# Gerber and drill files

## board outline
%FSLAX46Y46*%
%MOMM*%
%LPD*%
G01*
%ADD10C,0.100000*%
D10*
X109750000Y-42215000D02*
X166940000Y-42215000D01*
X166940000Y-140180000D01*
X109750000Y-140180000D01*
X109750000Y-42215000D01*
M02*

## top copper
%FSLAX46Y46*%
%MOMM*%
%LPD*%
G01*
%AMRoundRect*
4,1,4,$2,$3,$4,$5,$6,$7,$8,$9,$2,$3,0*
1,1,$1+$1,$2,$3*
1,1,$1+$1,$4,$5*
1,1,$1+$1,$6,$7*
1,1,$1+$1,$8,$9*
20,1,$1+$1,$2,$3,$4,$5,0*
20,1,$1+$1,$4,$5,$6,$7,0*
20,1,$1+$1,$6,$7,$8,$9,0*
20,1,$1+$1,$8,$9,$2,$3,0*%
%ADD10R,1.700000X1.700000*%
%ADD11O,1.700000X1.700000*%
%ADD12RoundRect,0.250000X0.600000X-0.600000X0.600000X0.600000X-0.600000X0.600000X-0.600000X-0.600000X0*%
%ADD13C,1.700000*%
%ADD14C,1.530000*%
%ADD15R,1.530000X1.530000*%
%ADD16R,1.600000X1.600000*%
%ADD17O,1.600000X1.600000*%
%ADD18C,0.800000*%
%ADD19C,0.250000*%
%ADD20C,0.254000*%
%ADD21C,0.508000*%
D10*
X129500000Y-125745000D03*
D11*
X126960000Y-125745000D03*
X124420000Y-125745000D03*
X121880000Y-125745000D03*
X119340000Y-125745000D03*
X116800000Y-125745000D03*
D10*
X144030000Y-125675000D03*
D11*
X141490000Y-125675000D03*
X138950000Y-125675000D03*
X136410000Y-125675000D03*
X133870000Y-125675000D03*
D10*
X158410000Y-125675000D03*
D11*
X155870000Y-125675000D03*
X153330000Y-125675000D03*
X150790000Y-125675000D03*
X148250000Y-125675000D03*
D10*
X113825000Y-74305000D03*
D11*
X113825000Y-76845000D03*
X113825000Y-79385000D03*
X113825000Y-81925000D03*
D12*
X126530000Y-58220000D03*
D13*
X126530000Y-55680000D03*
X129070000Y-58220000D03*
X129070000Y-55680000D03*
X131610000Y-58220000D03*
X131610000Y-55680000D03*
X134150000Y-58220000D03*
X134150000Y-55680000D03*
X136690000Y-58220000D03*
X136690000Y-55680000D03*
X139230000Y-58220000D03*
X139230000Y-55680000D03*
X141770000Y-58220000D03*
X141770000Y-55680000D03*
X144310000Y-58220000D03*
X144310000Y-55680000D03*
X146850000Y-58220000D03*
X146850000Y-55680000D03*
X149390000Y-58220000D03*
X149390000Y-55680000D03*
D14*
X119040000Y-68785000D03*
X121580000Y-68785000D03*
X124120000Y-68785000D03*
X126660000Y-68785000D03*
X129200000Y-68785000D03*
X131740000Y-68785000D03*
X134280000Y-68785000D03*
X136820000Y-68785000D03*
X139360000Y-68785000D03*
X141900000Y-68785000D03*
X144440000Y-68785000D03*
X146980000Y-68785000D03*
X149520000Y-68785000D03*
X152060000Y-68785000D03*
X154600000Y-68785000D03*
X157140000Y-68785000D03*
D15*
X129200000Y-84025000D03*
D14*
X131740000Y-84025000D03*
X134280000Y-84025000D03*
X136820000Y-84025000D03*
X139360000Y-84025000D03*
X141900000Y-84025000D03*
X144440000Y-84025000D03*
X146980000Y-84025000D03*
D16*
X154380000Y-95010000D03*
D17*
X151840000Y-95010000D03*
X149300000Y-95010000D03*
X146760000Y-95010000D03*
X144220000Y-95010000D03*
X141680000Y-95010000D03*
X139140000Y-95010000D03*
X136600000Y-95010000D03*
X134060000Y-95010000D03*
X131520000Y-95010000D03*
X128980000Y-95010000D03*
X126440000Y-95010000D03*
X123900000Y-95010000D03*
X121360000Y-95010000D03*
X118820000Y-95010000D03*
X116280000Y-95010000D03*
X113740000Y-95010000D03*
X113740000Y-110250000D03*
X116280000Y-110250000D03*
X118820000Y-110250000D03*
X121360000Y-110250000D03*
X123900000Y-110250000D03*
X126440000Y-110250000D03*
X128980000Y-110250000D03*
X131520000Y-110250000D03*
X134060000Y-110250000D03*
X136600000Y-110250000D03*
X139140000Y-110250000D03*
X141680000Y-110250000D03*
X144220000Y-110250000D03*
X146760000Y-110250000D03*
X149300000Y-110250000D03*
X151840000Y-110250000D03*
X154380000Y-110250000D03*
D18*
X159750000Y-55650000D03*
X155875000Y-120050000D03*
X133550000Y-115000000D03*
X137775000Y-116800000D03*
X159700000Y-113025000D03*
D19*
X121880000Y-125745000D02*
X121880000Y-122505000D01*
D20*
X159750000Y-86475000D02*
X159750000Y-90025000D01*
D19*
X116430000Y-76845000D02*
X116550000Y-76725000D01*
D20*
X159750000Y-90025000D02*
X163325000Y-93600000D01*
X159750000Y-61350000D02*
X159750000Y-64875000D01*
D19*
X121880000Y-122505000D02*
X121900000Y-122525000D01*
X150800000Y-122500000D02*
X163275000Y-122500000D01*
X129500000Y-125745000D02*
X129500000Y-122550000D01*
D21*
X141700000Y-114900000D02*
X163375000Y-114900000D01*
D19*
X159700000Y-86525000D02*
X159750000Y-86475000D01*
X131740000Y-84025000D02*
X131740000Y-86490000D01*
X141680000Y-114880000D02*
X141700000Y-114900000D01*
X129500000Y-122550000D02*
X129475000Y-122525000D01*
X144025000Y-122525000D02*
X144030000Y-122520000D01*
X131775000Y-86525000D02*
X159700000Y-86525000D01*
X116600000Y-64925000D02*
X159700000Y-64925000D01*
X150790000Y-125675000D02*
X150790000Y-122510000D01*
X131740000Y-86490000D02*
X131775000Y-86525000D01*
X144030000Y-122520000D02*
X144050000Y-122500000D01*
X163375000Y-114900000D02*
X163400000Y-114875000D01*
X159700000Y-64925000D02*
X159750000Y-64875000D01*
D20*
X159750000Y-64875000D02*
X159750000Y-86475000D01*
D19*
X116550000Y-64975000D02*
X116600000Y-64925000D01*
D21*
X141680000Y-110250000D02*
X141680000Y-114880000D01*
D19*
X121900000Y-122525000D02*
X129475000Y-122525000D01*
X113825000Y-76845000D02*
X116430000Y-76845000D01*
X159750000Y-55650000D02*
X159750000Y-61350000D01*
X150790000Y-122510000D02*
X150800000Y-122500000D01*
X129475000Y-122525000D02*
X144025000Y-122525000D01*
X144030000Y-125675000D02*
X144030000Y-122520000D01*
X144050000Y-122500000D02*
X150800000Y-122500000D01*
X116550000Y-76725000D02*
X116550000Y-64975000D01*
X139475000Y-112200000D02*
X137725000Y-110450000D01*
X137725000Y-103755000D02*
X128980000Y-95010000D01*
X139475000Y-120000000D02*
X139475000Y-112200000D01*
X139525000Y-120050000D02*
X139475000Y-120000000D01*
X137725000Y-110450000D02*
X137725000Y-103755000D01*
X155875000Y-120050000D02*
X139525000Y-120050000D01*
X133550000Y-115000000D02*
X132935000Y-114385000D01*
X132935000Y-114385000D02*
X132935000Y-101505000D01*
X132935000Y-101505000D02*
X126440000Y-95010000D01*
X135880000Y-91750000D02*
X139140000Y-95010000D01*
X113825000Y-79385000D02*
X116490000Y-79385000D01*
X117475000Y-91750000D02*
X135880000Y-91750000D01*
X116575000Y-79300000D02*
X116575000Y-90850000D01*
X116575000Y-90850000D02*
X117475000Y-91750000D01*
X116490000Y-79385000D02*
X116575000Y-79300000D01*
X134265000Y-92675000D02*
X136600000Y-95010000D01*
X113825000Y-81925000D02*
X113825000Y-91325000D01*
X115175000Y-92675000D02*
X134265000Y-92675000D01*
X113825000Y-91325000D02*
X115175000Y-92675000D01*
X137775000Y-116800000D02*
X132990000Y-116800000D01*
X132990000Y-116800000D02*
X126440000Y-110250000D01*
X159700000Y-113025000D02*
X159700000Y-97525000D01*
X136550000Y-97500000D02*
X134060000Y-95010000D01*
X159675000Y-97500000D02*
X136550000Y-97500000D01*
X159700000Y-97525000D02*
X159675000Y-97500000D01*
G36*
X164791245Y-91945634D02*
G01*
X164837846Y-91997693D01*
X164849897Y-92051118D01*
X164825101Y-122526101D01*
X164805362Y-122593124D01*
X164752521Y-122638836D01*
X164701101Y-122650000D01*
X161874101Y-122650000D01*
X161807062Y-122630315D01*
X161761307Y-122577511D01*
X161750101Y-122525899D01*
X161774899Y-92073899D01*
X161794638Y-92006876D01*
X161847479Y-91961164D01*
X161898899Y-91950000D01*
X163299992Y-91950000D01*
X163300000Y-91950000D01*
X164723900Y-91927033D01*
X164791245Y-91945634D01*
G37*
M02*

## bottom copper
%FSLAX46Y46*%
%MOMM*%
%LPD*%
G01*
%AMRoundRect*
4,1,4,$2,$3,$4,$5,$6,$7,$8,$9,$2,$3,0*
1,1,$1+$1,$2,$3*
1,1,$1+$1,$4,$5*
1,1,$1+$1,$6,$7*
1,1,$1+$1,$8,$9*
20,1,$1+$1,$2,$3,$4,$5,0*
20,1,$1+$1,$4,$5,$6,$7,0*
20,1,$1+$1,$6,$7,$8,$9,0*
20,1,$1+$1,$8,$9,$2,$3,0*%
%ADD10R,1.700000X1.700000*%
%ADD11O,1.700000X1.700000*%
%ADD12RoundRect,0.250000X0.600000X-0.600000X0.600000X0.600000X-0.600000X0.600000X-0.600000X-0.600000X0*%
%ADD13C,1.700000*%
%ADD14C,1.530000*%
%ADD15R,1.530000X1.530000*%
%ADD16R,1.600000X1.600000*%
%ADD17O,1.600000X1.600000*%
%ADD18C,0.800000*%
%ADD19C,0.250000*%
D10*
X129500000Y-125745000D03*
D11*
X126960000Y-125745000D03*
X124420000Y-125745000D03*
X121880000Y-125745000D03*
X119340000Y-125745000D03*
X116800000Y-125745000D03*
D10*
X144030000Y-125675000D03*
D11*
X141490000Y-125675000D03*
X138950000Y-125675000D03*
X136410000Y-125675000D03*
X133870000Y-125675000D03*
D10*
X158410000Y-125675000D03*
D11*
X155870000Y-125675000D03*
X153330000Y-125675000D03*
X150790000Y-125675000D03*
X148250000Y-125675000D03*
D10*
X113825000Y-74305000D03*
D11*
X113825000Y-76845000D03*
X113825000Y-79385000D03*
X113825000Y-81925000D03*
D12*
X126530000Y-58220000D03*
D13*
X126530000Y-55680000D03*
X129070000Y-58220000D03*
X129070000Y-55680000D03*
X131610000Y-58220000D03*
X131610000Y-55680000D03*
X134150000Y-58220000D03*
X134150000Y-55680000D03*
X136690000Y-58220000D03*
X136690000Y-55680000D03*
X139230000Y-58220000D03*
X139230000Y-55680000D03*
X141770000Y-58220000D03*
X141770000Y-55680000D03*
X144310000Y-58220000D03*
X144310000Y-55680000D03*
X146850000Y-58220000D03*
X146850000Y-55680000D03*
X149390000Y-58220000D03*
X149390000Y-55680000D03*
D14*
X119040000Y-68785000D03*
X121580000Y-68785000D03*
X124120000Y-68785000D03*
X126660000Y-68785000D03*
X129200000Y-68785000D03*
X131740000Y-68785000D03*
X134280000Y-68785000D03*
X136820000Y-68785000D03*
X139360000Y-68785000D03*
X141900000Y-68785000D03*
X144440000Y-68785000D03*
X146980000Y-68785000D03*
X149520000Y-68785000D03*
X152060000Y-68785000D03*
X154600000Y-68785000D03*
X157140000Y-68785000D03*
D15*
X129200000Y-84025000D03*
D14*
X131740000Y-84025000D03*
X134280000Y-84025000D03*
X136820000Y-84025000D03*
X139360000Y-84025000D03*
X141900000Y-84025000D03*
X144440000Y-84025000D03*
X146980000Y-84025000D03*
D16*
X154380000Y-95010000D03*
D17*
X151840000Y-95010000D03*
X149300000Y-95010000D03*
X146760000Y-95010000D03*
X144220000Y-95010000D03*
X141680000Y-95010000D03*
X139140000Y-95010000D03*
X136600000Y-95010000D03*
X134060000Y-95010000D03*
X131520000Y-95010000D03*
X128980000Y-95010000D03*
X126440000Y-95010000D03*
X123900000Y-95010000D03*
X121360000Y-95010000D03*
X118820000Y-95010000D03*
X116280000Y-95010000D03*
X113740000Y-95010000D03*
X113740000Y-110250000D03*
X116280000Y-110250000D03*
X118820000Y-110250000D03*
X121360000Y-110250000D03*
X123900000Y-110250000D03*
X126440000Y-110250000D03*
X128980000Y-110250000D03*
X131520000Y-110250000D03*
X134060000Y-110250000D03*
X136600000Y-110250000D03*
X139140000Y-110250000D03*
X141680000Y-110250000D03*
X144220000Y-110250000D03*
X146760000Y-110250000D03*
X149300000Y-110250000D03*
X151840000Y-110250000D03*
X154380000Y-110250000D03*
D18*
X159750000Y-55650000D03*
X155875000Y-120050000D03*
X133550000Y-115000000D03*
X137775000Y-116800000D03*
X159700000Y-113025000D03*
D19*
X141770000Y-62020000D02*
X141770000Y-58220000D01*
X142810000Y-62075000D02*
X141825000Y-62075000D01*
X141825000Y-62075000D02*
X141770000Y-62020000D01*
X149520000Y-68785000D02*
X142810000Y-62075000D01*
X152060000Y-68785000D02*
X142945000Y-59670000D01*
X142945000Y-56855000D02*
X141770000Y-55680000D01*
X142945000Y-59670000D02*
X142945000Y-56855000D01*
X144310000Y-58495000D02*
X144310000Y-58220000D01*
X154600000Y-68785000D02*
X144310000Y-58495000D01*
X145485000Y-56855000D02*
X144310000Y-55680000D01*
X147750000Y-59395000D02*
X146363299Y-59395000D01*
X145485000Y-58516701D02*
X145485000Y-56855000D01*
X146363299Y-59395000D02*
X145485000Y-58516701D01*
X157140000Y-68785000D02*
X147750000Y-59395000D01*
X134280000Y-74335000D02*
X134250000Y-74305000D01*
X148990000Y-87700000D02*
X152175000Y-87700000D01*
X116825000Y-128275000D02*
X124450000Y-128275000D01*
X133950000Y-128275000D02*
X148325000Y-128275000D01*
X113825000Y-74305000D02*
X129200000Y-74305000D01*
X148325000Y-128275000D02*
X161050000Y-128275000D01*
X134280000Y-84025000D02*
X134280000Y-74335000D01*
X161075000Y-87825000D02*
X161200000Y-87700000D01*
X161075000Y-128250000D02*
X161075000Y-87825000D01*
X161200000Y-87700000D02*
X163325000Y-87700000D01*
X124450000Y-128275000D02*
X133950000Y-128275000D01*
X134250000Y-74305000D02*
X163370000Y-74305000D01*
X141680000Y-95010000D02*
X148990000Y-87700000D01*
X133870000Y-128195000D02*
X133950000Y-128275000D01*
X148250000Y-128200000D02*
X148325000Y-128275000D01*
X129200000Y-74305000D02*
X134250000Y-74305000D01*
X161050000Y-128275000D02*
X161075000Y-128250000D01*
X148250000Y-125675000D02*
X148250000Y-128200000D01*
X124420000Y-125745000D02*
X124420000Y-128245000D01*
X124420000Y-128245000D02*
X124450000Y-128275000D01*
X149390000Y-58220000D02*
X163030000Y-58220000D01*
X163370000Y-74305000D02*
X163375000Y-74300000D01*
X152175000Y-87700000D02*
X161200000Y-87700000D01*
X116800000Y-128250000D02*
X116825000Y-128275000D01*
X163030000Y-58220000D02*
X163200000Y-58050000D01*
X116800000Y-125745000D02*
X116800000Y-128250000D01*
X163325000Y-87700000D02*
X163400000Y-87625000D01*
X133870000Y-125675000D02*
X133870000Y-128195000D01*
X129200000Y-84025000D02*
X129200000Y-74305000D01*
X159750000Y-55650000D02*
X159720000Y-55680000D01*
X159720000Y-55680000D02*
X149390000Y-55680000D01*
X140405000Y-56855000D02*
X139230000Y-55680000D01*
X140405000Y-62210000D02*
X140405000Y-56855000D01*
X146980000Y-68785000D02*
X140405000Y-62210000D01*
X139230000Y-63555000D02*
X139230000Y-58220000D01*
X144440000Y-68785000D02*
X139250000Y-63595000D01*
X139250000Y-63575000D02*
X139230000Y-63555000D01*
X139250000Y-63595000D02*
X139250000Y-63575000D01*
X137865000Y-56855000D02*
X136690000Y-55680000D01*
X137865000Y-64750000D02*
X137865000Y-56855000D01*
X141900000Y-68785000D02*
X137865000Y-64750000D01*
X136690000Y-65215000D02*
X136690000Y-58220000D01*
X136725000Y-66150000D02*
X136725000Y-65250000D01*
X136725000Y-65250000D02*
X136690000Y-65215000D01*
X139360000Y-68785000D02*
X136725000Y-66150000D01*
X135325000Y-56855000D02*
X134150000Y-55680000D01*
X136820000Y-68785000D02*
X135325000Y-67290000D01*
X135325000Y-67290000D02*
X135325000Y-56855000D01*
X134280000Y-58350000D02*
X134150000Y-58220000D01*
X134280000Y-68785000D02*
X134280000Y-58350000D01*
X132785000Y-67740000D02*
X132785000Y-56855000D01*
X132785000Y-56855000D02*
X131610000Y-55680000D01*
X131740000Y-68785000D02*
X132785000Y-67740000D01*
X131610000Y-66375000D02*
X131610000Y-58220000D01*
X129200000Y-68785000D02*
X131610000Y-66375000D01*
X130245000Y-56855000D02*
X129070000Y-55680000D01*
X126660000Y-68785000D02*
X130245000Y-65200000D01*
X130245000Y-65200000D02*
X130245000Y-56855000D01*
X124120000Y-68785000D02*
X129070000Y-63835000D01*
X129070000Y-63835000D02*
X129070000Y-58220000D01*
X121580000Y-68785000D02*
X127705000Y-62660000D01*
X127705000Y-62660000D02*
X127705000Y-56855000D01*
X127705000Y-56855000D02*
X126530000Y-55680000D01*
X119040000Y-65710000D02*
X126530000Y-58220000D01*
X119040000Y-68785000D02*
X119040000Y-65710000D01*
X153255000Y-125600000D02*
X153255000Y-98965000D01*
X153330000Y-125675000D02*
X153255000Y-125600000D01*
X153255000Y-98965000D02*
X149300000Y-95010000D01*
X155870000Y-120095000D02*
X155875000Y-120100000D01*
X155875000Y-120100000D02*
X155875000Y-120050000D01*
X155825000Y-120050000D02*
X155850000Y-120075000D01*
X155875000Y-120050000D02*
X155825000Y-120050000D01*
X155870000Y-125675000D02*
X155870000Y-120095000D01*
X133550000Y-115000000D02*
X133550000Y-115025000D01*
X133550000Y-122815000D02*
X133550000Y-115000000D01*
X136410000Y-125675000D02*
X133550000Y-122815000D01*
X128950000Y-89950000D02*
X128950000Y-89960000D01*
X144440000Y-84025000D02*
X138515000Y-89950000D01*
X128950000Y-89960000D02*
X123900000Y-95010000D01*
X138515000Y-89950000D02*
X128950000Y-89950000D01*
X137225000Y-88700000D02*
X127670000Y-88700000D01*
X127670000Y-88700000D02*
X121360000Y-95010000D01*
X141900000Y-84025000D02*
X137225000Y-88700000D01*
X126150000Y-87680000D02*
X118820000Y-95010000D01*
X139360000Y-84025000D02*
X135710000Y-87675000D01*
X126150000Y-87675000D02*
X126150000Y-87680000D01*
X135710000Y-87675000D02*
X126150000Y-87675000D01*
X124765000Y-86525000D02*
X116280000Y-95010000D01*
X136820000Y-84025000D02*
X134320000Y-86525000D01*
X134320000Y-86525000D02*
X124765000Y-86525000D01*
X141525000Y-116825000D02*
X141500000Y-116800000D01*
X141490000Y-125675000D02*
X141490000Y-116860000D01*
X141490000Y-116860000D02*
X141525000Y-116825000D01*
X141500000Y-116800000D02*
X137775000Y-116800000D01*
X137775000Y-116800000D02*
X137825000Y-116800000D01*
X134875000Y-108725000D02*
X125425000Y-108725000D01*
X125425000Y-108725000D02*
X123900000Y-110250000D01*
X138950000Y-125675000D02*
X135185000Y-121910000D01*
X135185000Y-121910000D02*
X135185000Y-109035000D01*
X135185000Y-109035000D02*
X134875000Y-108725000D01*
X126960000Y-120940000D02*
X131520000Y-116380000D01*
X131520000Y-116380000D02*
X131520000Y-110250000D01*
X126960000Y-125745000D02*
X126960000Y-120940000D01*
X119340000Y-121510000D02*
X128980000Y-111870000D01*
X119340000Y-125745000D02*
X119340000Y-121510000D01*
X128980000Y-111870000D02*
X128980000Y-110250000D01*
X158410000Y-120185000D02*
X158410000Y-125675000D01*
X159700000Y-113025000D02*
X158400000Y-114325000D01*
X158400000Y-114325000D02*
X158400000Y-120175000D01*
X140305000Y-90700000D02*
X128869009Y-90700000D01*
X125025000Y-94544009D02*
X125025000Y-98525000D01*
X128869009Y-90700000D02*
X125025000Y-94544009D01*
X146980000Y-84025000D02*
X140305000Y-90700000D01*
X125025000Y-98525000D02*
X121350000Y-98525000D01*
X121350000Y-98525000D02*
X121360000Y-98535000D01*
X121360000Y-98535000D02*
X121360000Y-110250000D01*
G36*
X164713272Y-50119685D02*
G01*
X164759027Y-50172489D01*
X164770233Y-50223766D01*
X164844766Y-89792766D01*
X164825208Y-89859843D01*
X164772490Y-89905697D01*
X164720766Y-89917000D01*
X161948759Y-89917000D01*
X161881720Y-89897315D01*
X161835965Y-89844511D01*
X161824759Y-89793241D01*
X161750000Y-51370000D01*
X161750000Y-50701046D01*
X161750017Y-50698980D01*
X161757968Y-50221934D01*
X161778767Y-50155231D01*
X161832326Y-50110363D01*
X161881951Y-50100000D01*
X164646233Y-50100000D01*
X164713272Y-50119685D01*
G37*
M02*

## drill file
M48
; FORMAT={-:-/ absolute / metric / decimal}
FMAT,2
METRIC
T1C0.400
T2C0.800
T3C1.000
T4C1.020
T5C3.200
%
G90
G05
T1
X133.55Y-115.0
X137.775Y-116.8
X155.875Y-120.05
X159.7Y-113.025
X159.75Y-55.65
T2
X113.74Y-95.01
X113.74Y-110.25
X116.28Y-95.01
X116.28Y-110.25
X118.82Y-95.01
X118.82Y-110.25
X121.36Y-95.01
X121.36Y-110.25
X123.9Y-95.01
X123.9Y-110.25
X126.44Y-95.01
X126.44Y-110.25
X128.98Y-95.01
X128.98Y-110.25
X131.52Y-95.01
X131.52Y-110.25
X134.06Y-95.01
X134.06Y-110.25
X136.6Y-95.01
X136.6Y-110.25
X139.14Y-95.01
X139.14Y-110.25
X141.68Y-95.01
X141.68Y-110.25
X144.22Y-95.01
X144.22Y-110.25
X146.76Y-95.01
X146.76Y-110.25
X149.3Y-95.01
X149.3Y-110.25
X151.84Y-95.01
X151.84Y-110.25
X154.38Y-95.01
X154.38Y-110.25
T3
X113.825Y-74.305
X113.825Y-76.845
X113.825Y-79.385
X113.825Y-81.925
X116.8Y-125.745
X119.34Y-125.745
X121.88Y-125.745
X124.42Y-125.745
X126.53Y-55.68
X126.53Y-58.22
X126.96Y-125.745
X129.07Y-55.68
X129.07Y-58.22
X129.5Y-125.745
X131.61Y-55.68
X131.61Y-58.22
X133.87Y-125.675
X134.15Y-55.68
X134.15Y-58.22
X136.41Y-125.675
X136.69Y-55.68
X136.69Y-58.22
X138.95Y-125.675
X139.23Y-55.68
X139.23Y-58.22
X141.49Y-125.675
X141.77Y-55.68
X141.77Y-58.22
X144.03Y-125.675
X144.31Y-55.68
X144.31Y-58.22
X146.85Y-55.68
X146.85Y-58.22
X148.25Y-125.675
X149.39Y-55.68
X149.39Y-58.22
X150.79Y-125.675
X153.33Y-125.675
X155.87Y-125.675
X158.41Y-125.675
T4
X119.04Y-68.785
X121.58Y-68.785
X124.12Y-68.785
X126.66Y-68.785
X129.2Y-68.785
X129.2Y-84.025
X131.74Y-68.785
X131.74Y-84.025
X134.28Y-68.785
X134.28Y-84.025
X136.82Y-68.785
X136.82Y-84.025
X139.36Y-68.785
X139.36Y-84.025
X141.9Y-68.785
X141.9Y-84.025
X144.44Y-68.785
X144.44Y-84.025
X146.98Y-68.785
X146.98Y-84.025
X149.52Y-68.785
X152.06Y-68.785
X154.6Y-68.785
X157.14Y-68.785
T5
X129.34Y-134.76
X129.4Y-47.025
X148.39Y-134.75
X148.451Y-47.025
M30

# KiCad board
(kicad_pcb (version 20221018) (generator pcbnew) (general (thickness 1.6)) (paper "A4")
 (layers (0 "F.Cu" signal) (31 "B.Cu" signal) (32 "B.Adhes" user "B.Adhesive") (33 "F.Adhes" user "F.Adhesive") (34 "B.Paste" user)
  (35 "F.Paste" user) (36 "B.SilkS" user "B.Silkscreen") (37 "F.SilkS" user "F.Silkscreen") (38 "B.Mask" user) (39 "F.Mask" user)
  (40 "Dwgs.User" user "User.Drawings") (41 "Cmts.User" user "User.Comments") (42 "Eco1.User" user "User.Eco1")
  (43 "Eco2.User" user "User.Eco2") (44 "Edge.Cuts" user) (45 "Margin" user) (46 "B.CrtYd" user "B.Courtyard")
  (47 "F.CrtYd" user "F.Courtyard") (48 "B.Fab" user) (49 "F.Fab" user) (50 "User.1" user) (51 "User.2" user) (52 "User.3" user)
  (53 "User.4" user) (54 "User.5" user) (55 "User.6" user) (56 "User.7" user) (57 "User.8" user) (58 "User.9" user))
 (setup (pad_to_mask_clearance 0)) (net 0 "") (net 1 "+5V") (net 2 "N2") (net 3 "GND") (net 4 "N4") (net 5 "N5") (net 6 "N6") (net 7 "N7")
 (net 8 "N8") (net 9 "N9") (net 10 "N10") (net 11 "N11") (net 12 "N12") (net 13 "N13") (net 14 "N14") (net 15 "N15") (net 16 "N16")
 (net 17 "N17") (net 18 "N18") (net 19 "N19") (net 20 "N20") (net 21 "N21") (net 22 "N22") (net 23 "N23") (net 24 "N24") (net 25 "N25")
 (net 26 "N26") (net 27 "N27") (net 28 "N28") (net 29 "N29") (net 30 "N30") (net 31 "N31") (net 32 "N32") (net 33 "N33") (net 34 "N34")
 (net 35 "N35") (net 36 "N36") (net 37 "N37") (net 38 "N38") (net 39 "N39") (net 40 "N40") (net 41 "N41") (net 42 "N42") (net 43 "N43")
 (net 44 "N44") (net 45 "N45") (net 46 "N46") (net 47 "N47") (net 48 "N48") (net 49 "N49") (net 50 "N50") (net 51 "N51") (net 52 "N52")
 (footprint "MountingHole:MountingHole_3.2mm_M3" (layer "F.Cu") (at 129.4 47.025)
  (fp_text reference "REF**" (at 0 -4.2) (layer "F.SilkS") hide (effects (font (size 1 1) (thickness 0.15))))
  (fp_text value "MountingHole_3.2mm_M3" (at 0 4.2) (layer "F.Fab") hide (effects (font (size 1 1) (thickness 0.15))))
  (pad "" np_thru_hole circle (at 0 0) (size 3.2 3.2) (drill 3.2) (layers "*.Cu" "*.Mask")))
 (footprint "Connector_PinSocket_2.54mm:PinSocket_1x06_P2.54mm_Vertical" (layer "F.Cu") (at 129.5 125.745 -90)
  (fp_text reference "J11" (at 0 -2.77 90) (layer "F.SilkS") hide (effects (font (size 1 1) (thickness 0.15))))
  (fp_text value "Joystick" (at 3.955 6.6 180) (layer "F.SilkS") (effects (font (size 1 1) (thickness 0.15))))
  (pad "1" thru_hole rect (at 0 0 270) (size 1.7 1.7) (drill 1) (layers "*.Cu" "*.Mask") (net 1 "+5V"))
  (pad "2" thru_hole oval (at 0 2.54 270) (size 1.7 1.7) (drill 1) (layers "*.Cu" "*.Mask") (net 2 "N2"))
  (pad "3" thru_hole oval (at 0 5.08 270) (size 1.7 1.7) (drill 1) (layers "*.Cu" "*.Mask") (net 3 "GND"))
  (pad "4" thru_hole oval (at 0 7.62 270) (size 1.7 1.7) (drill 1) (layers "*.Cu" "*.Mask") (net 1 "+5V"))
  (pad "5" thru_hole oval (at 0 10.16 270) (size 1.7 1.7) (drill 1) (layers "*.Cu" "*.Mask") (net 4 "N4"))
  (pad "6" thru_hole oval (at 0 12.7 270) (size 1.7 1.7) (drill 1) (layers "*.Cu" "*.Mask") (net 3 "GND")))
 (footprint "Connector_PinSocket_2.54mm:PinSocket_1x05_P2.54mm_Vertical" (layer "F.Cu") (at 144.03 125.675 -90)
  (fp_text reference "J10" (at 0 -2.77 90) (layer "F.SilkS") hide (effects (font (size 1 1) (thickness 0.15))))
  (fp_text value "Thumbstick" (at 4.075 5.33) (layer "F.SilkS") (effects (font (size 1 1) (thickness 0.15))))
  (pad "1" thru_hole rect (at 0 0 270) (size 1.7 1.7) (drill 1) (layers "*.Cu" "*.Mask") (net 1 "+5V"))
  (pad "2" thru_hole oval (at 0 2.54 270) (size 1.7 1.7) (drill 1) (layers "*.Cu" "*.Mask") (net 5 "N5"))
  (pad "3" thru_hole oval (at 0 5.08 270) (size 1.7 1.7) (drill 1) (layers "*.Cu" "*.Mask") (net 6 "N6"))
  (pad "4" thru_hole oval (at 0 7.62 270) (size 1.7 1.7) (drill 1) (layers "*.Cu" "*.Mask") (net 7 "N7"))
  (pad "5" thru_hole oval (at 0 10.16 270) (size 1.7 1.7) (drill 1) (layers "*.Cu" "*.Mask") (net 3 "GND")))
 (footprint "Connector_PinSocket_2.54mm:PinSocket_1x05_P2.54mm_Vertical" (layer "F.Cu") (at 158.41 125.675 -90)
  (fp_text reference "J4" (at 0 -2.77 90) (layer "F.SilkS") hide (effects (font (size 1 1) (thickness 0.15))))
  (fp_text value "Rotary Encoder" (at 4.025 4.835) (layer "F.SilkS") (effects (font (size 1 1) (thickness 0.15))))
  (pad "1" thru_hole rect (at 0 0 270) (size 1.7 1.7) (drill 1) (layers "*.Cu" "*.Mask") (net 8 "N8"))
  (pad "2" thru_hole oval (at 0 2.54 270) (size 1.7 1.7) (drill 1) (layers "*.Cu" "*.Mask") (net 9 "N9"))
  (pad "3" thru_hole oval (at 0 5.08 270) (size 1.7 1.7) (drill 1) (layers "*.Cu" "*.Mask") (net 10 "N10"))
  (pad "4" thru_hole oval (at 0 7.62 270) (size 1.7 1.7) (drill 1) (layers "*.Cu" "*.Mask") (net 1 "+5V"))
  (pad "5" thru_hole oval (at 0 10.16 270) (size 1.7 1.7) (drill 1) (layers "*.Cu" "*.Mask") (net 3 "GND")))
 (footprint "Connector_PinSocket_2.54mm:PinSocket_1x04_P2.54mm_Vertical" (layer "F.Cu") (at 113.825 74.305)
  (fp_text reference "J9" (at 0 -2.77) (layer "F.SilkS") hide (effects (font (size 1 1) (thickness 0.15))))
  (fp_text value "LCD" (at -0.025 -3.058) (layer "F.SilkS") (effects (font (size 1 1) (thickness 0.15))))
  (pad "1" thru_hole rect (at 0 0) (size 1.7 1.7) (drill 1) (layers "*.Cu" "*.Mask") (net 3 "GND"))
  (pad "2" thru_hole oval (at 0 2.54) (size 1.7 1.7) (drill 1) (layers "*.Cu" "*.Mask") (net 1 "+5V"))
  (pad "3" thru_hole oval (at 0 5.08) (size 1.7 1.7) (drill 1) (layers "*.Cu" "*.Mask") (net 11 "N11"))
  (pad "4" thru_hole oval (at 0 7.62) (size 1.7 1.7) (drill 1) (layers "*.Cu" "*.Mask") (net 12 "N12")))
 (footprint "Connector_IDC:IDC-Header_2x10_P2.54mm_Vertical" (layer "F.Cu") (at 126.53 58.22 90)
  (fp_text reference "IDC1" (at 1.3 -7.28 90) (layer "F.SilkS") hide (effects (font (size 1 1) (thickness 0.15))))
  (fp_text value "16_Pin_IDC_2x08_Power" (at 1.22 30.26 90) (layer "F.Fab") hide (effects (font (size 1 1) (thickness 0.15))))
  (pad "1" thru_hole roundrect (at 0 0 90) (size 1.7 1.7) (drill 1) (layers "*.Cu" "*.Mask") (roundrect_rratio 0.1470588235) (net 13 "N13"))
  (pad "2" thru_hole circle (at 2.54 0 90) (size 1.7 1.7) (drill 1) (layers "*.Cu" "*.Mask") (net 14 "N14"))
  (pad "3" thru_hole circle (at 0 2.54 90) (size 1.7 1.7) (drill 1) (layers "*.Cu" "*.Mask") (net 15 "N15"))
  (pad "4" thru_hole circle (at 2.54 2.54 90) (size 1.7 1.7) (drill 1) (layers "*.Cu" "*.Mask") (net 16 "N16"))
  (pad "5" thru_hole circle (at 0 5.08 90) (size 1.7 1.7) (drill 1) (layers "*.Cu" "*.Mask") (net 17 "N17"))
  (pad "6" thru_hole circle (at 2.54 5.08 90) (size 1.7 1.7) (drill 1) (layers "*.Cu" "*.Mask") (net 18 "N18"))
  (pad "7" thru_hole circle (at 0 7.62 90) (size 1.7 1.7) (drill 1) (layers "*.Cu" "*.Mask") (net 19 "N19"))
  (pad "8" thru_hole circle (at 2.54 7.62 90) (size 1.7 1.7) (drill 1) (layers "*.Cu" "*.Mask") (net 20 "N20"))
  (pad "9" thru_hole circle (at 0 10.16 90) (size 1.7 1.7) (drill 1) (layers "*.Cu" "*.Mask") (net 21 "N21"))
  (pad "10" thru_hole circle (at 2.54 10.16 90) (size 1.7 1.7) (drill 1) (layers "*.Cu" "*.Mask") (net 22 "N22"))
  (pad "11" thru_hole circle (at 0 12.7 90) (size 1.7 1.7) (drill 1) (layers "*.Cu" "*.Mask") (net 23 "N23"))
  (pad "12" thru_hole circle (at 2.54 12.7 90) (size 1.7 1.7) (drill 1) (layers "*.Cu" "*.Mask") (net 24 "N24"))
  (pad "13" thru_hole circle (at 0 15.24 90) (size 1.7 1.7) (drill 1) (layers "*.Cu" "*.Mask") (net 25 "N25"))
  (pad "14" thru_hole circle (at 2.54 15.24 90) (size 1.7 1.7) (drill 1) (layers "*.Cu" "*.Mask") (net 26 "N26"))
  (pad "15" thru_hole circle (at 0 17.78 90) (size 1.7 1.7) (drill 1) (layers "*.Cu" "*.Mask") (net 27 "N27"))
  (pad "16" thru_hole circle (at 2.54 17.78 90) (size 1.7 1.7) (drill 1) (layers "*.Cu" "*.Mask") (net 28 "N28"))
  (pad "17" thru_hole circle (at 0 20.32 90) (size 1.7 1.7) (drill 1) (layers "*.Cu" "*.Mask") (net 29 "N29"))
  (pad "18" thru_hole circle (at 2.54 20.32 90) (size 1.7 1.7) (drill 1) (layers "*.Cu" "*.Mask") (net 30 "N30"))
  (pad "19" thru_hole circle (at 0 22.86 90) (size 1.7 1.7) (drill 1) (layers "*.Cu" "*.Mask") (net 3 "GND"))
  (pad "20" thru_hole circle (at 2.54 22.86 90) (size 1.7 1.7) (drill 1) (layers "*.Cu" "*.Mask") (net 1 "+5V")))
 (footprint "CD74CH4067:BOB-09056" (layer "F.Cu") (at 138.09 76.405 -90)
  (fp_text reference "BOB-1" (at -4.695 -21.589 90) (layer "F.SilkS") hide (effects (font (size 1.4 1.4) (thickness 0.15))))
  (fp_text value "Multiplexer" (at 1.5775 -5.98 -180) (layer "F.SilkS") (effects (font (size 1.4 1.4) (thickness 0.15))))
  (pad "JP1-1" thru_hole circle (at -7.62 19.05 270) (size 1.53 1.53) (drill 1.02) (layers "*.Cu" "*.Mask") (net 13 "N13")
   (solder_mask_margin 0.102))
  (pad "JP1-2" thru_hole circle (at -7.62 16.51 270) (size 1.53 1.53) (drill 1.02) (layers "*.Cu" "*.Mask") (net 14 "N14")
   (solder_mask_margin 0.102))
  (pad "JP1-3" thru_hole circle (at -7.62 13.97 270) (size 1.53 1.53) (drill 1.02) (layers "*.Cu" "*.Mask") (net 15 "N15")
   (solder_mask_margin 0.102))
  (pad "JP1-4" thru_hole circle (at -7.62 11.43 270) (size 1.53 1.53) (drill 1.02) (layers "*.Cu" "*.Mask") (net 16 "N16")
   (solder_mask_margin 0.102))
  (pad "JP1-5" thru_hole circle (at -7.62 8.89 270) (size 1.53 1.53) (drill 1.02) (layers "*.Cu" "*.Mask") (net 17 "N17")
   (solder_mask_margin 0.102))
  (pad "JP1-6" thru_hole circle (at -7.62 6.35 270) (size 1.53 1.53) (drill 1.02) (layers "*.Cu" "*.Mask") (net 18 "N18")
   (solder_mask_margin 0.102))
  (pad "JP1-7" thru_hole circle (at -7.62 3.81 270) (size 1.53 1.53) (drill 1.02) (layers "*.Cu" "*.Mask") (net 19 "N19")
   (solder_mask_margin 0.102))
  (pad "JP1-8" thru_hole circle (at -7.62 1.27 270) (size 1.53 1.53) (drill 1.02) (layers "*.Cu" "*.Mask") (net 20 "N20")
   (solder_mask_margin 0.102))
  (pad "JP1-9" thru_hole circle (at -7.62 -1.27 270) (size 1.53 1.53) (drill 1.02) (layers "*.Cu" "*.Mask") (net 21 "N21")
   (solder_mask_margin 0.102))
  (pad "JP1-10" thru_hole circle (at -7.62 -3.81 270) (size 1.53 1.53) (drill 1.02) (layers "*.Cu" "*.Mask") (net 22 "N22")
   (solder_mask_margin 0.102))
  (pad "JP1-11" thru_hole circle (at -7.62 -6.35 270) (size 1.53 1.53) (drill 1.02) (layers "*.Cu" "*.Mask") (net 23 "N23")
   (solder_mask_margin 0.102))
  (pad "JP1-12" thru_hole circle (at -7.62 -8.89 270) (size 1.53 1.53) (drill 1.02) (layers "*.Cu" "*.Mask") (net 24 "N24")
   (solder_mask_margin 0.102))
  (pad "JP1-13" thru_hole circle (at -7.62 -11.43 270) (size 1.53 1.53) (drill 1.02) (layers "*.Cu" "*.Mask") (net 25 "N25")
   (solder_mask_margin 0.102))
  (pad "JP1-14" thru_hole circle (at -7.62 -13.97 270) (size 1.53 1.53) (drill 1.02) (layers "*.Cu" "*.Mask") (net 26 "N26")
   (solder_mask_margin 0.102))
  (pad "JP1-15" thru_hole circle (at -7.62 -16.51 270) (size 1.53 1.53) (drill 1.02) (layers "*.Cu" "*.Mask") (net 27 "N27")
   (solder_mask_margin 0.102))
  (pad "JP1-16" thru_hole circle (at -7.62 -19.05 270) (size 1.53 1.53) (drill 1.02) (layers "*.Cu" "*.Mask") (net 28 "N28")
   (solder_mask_margin 0.102))
  (pad "JP3-1" thru_hole rect (at 7.62 8.89 270) (size 1.53 1.53) (drill 1.02) (layers "*.Cu" "*.Mask") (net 3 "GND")
   (solder_mask_margin 0.102))
  (pad "JP3-2" thru_hole circle (at 7.62 6.35 270) (size 1.53 1.53) (drill 1.02) (layers "*.Cu" "*.Mask") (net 1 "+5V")
   (solder_mask_margin 0.102))
  (pad "JP3-3" thru_hole circle (at 7.62 3.81 270) (size 1.53 1.53) (drill 1.02) (layers "*.Cu" "*.Mask") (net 3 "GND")
   (solder_mask_margin 0.102))
  (pad "JP3-4" thru_hole circle (at 7.62 1.27 270) (size 1.53 1.53) (drill 1.02) (layers "*.Cu" "*.Mask") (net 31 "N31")
   (solder_mask_margin 0.102))
  (pad "JP3-5" thru_hole circle (at 7.62 -1.27 270) (size 1.53 1.53) (drill 1.02) (layers "*.Cu" "*.Mask") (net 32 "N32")
   (solder_mask_margin 0.102))
  (pad "JP3-6" thru_hole circle (at 7.62 -3.81 270) (size 1.53 1.53) (drill 1.02) (layers "*.Cu" "*.Mask") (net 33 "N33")
   (solder_mask_margin 0.102))
  (pad "JP3-7" thru_hole circle (at 7.62 -6.35 270) (size 1.53 1.53) (drill 1.02) (layers "*.Cu" "*.Mask") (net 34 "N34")
   (solder_mask_margin 0.102))
  (pad "JP3-8" thru_hole circle (at 7.62 -8.89 270) (size 1.53 1.53) (drill 1.02) (layers "*.Cu" "*.Mask") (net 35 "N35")
   (solder_mask_margin 0.102)))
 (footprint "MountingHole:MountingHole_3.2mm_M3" (layer "F.Cu") (at 129.34 134.76)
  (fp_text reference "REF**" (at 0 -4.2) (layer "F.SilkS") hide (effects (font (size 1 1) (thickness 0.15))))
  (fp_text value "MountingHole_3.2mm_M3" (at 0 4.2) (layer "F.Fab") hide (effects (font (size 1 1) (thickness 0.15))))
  (pad "" np_thru_hole circle (at 0 0) (size 3.2 3.2) (drill 3.2) (layers "*.Cu" "*.Mask")))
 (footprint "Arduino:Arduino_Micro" (layer "F.Cu") (at 154.38 95.01 -90)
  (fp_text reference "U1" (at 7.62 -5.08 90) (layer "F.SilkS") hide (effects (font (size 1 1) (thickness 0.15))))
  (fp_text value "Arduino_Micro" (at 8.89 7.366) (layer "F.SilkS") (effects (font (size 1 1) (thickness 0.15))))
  (pad "1" thru_hole rect (at 0 0 270) (size 1.6 1.6) (drill 0.8) (layers "*.Cu" "*.Mask") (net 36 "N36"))
  (pad "2" thru_hole oval (at 0 2.54 270) (size 1.6 1.6) (drill 0.8) (layers "*.Cu" "*.Mask") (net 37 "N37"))
  (pad "3" thru_hole oval (at 0 5.08 270) (size 1.6 1.6) (drill 0.8) (layers "*.Cu" "*.Mask") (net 10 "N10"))
  (pad "4" thru_hole oval (at 0 7.62 270) (size 1.6 1.6) (drill 0.8) (layers "*.Cu" "*.Mask") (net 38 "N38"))
  (pad "5" thru_hole oval (at 0 10.16 270) (size 1.6 1.6) (drill 0.8) (layers "*.Cu" "*.Mask") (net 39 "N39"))
  (pad "6" thru_hole oval (at 0 12.7 270) (size 1.6 1.6) (drill 0.8) (layers "*.Cu" "*.Mask") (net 3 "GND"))
  (pad "7" thru_hole oval (at 0 15.24 270) (size 1.6 1.6) (drill 0.8) (layers "*.Cu" "*.Mask") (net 11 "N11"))
  (pad "8" thru_hole oval (at 0 17.78 270) (size 1.6 1.6) (drill 0.8) (layers "*.Cu" "*.Mask") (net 12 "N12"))
  (pad "9" thru_hole oval (at 0 20.32 270) (size 1.6 1.6) (drill 0.8) (layers "*.Cu" "*.Mask") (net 8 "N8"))
  (pad "10" thru_hole oval (at 0 22.86 270) (size 1.6 1.6) (drill 0.8) (layers "*.Cu" "*.Mask") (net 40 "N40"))
  (pad "11" thru_hole oval (at 0 25.4 270) (size 1.6 1.6) (drill 0.8) (layers "*.Cu" "*.Mask") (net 9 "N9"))
  (pad "12" thru_hole oval (at 0 27.94 270) (size 1.6 1.6) (drill 0.8) (layers "*.Cu" "*.Mask") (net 7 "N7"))
  (pad "13" thru_hole oval (at 0 30.48 270) (size 1.6 1.6) (drill 0.8) (layers "*.Cu" "*.Mask") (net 34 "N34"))
  (pad "14" thru_hole oval (at 0 33.02 270) (size 1.6 1.6) (drill 0.8) (layers "*.Cu" "*.Mask") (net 33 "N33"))
  (pad "15" thru_hole oval (at 0 35.56 270) (size 1.6 1.6) (drill 0.8) (layers "*.Cu" "*.Mask") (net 32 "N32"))
  (pad "16" thru_hole oval (at 0 38.1 270) (size 1.6 1.6) (drill 0.8) (layers "*.Cu" "*.Mask") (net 31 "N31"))
  (pad "17" thru_hole oval (at 0 40.64 270) (size 1.6 1.6) (drill 0.8) (layers "*.Cu" "*.Mask") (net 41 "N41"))
  (pad "18" thru_hole oval (at 15.24 40.64 270) (size 1.6 1.6) (drill 0.8) (layers "*.Cu" "*.Mask") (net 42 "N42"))
  (pad "19" thru_hole oval (at 15.24 38.1 270) (size 1.6 1.6) (drill 0.8) (layers "*.Cu" "*.Mask") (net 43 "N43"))
  (pad "20" thru_hole oval (at 15.24 35.56 270) (size 1.6 1.6) (drill 0.8) (layers "*.Cu" "*.Mask") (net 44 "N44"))
  (pad "21" thru_hole oval (at 15.24 33.02 270) (size 1.6 1.6) (drill 0.8) (layers "*.Cu" "*.Mask") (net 35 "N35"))
  (pad "22" thru_hole oval (at 15.24 30.48 270) (size 1.6 1.6) (drill 0.8) (layers "*.Cu" "*.Mask") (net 6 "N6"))
  (pad "23" thru_hole oval (at 15.24 27.94 270) (size 1.6 1.6) (drill 0.8) (layers "*.Cu" "*.Mask") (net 5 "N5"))
  (pad "24" thru_hole oval (at 15.24 25.4 270) (size 1.6 1.6) (drill 0.8) (layers "*.Cu" "*.Mask") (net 4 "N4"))
  (pad "25" thru_hole oval (at 15.24 22.86 270) (size 1.6 1.6) (drill 0.8) (layers "*.Cu" "*.Mask") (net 2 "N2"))
  (pad "26" thru_hole oval (at 15.24 20.32 270) (size 1.6 1.6) (drill 0.8) (layers "*.Cu" "*.Mask") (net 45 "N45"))
  (pad "27" thru_hole oval (at 15.24 17.78 270) (size 1.6 1.6) (drill 0.8) (layers "*.Cu" "*.Mask") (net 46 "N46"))
  (pad "28" thru_hole oval (at 15.24 15.24 270) (size 1.6 1.6) (drill 0.8) (layers "*.Cu" "*.Mask") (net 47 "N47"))
  (pad "29" thru_hole oval (at 15.24 12.7 270) (size 1.6 1.6) (drill 0.8) (layers "*.Cu" "*.Mask") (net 1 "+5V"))
  (pad "30" thru_hole oval (at 15.24 10.16 270) (size 1.6 1.6) (drill 0.8) (layers "*.Cu" "*.Mask") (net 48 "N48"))
  (pad "31" thru_hole oval (at 15.24 7.62 270) (size 1.6 1.6) (drill 0.8) (layers "*.Cu" "*.Mask") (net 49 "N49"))
  (pad "32" thru_hole oval (at 15.24 5.08 270) (size 1.6 1.6) (drill 0.8) (layers "*.Cu" "*.Mask") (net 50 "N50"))
  (pad "33" thru_hole oval (at 15.24 2.54 270) (size 1.6 1.6) (drill 0.8) (layers "*.Cu" "*.Mask") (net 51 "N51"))
  (pad "34" thru_hole oval (at 15.24 0 270) (size 1.6 1.6) (drill 0.8) (layers "*.Cu" "*.Mask") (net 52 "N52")))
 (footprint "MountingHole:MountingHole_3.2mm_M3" (layer "F.Cu") (at 148.39 134.75)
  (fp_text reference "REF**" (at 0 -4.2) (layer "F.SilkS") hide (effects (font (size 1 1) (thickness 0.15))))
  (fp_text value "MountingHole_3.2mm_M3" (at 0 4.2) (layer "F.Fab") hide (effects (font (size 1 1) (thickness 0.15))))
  (pad "" np_thru_hole circle (at 0 0) (size 3.2 3.2) (drill 3.2) (layers "*.Cu" "*.Mask")))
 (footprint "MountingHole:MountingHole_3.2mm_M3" (layer "F.Cu") (at 148.451418 47.025)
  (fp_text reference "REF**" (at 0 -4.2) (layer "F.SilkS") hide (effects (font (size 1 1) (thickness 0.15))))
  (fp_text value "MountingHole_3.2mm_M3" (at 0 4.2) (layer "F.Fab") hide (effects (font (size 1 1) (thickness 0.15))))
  (pad "" np_thru_hole circle (at 0 0) (size 3.2 3.2) (drill 3.2) (layers "*.Cu" "*.Mask")))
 (gr_rect (start 109.75 42.215) (end 166.94 140.18) (stroke (width 0.1) (type default)) (fill none) (layer "Edge.Cuts"))
 (segment (start 141.77 62.02) (end 141.77 58.22) (width 0.25) (layer "B.Cu") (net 25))
 (segment (start 142.81 62.075) (end 141.825 62.075) (width 0.25) (layer "B.Cu") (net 25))
 (segment (start 141.825 62.075) (end 141.77 62.02) (width 0.25) (layer "B.Cu") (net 25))
 (segment (start 149.52 68.785) (end 142.81 62.075) (width 0.25) (layer "B.Cu") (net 25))
 (segment (start 152.06 68.785) (end 142.945 59.67) (width 0.25) (layer "B.Cu") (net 26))
 (segment (start 142.945 56.855) (end 141.77 55.68) (width 0.25) (layer "B.Cu") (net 26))
 (segment (start 142.945 59.67) (end 142.945 56.855) (width 0.25) (layer "B.Cu") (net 26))
 (segment (start 144.31 58.495) (end 144.31 58.22) (width 0.25) (layer "B.Cu") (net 27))
 (segment (start 154.6 68.785) (end 144.31 58.495) (width 0.25) (layer "B.Cu") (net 27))
 (segment (start 145.485 56.855) (end 144.31 55.68) (width 0.25) (layer "B.Cu") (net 28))
 (segment (start 147.75 59.395) (end 146.363299 59.395) (width 0.25) (layer "B.Cu") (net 28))
 (segment (start 145.485 58.516701) (end 145.485 56.855) (width 0.25) (layer "B.Cu") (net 28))
 (segment (start 146.363299 59.395) (end 145.485 58.516701) (width 0.25) (layer "B.Cu") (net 28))
 (segment (start 157.14 68.785) (end 147.75 59.395) (width 0.25) (layer "B.Cu") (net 28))
 (segment (start 134.28 74.335) (end 134.25 74.305) (width 0.25) (layer "B.Cu") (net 3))
 (segment (start 148.99 87.7) (end 152.175 87.7) (width 0.25) (layer "B.Cu") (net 3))
 (segment (start 116.825 128.275) (end 124.45 128.275) (width 0.25) (layer "B.Cu") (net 3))
 (segment (start 133.95 128.275) (end 148.325 128.275) (width 0.25) (layer "B.Cu") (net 3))
 (segment (start 113.825 74.305) (end 129.2 74.305) (width 0.25) (layer "B.Cu") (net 3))
 (segment (start 148.325 128.275) (end 161.05 128.275) (width 0.25) (layer "B.Cu") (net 3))
 (segment (start 134.28 84.025) (end 134.28 74.335) (width 0.25) (layer "B.Cu") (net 3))
 (segment (start 161.075 87.825) (end 161.2 87.7) (width 0.25) (layer "B.Cu") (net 3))
 (segment (start 161.075 128.25) (end 161.075 87.825) (width 0.25) (layer "B.Cu") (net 3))
 (segment (start 161.2 87.7) (end 163.325 87.7) (width 0.25) (layer "B.Cu") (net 3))
 (segment (start 124.45 128.275) (end 133.95 128.275) (width 0.25) (layer "B.Cu") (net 3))
 (segment (start 134.25 74.305) (end 163.37 74.305) (width 0.25) (layer "B.Cu") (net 3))
 (segment (start 141.68 95.01) (end 148.99 87.7) (width 0.25) (layer "B.Cu") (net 3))
 (segment (start 133.87 128.195) (end 133.95 128.275) (width 0.25) (layer "B.Cu") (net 3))
 (segment (start 148.25 128.2) (end 148.325 128.275) (width 0.25) (layer "B.Cu") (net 3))
 (segment (start 129.2 74.305) (end 134.25 74.305) (width 0.25) (layer "B.Cu") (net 3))
 (segment (start 161.05 128.275) (end 161.075 128.25) (width 0.25) (layer "B.Cu") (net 3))
 (segment (start 148.25 125.675) (end 148.25 128.2) (width 0.25) (layer "B.Cu") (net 3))
 (segment (start 124.42 125.745) (end 124.42 128.245) (width 0.25) (layer "B.Cu") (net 3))
 (segment (start 124.42 128.245) (end 124.45 128.275) (width 0.25) (layer "B.Cu") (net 3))
 (segment (start 149.39 58.22) (end 163.03 58.22) (width 0.25) (layer "B.Cu") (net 3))
 (segment (start 163.37 74.305) (end 163.375 74.3) (width 0.25) (layer "B.Cu") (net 3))
 (segment (start 152.175 87.7) (end 161.2 87.7) (width 0.25) (layer "B.Cu") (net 3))
 (segment (start 116.8 128.25) (end 116.825 128.275) (width 0.25) (layer "B.Cu") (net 3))
 (segment (start 163.03 58.22) (end 163.2 58.05) (width 0.25) (layer "B.Cu") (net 3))
 (segment (start 116.8 125.745) (end 116.8 128.25) (width 0.25) (layer "B.Cu") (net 3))
 (segment (start 163.325 87.7) (end 163.4 87.625) (width 0.25) (layer "B.Cu") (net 3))
 (segment (start 133.87 125.675) (end 133.87 128.195) (width 0.25) (layer "B.Cu") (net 3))
 (segment (start 129.2 84.025) (end 129.2 74.305) (width 0.25) (layer "B.Cu") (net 3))
 (segment (start 121.88 125.745) (end 121.88 122.505) (width 0.25) (layer "F.Cu") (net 1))
 (segment (start 159.75 86.475) (end 159.75 90.025) (width 0.254) (layer "F.Cu") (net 1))
 (segment (start 116.43 76.845) (end 116.55 76.725) (width 0.25) (layer "F.Cu") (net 1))
 (segment (start 159.75 90.025) (end 163.325 93.6) (width 0.254) (layer "F.Cu") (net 1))
 (segment (start 159.75 61.35) (end 159.75 64.875) (width 0.254) (layer "F.Cu") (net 1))
 (segment (start 121.88 122.505) (end 121.9 122.525) (width 0.25) (layer "F.Cu") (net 1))
 (segment (start 150.8 122.5) (end 163.275 122.5) (width 0.25) (layer "F.Cu") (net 1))
 (segment (start 129.5 125.745) (end 129.5 122.55) (width 0.25) (layer "F.Cu") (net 1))
 (segment (start 141.7 114.9) (end 163.375 114.9) (width 0.508) (layer "F.Cu") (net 1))
 (segment (start 159.7 86.525) (end 159.75 86.475) (width 0.25) (layer "F.Cu") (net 1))
 (segment (start 131.74 84.025) (end 131.74 86.49) (width 0.25) (layer "F.Cu") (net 1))
 (segment (start 141.68 114.88) (end 141.7 114.9) (width 0.25) (layer "F.Cu") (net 1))
 (segment (start 129.5 122.55) (end 129.475 122.525) (width 0.25) (layer "F.Cu") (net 1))
 (segment (start 144.025 122.525) (end 144.03 122.52) (width 0.25) (layer "F.Cu") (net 1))
 (segment (start 131.775 86.525) (end 159.7 86.525) (width 0.25) (layer "F.Cu") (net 1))
 (segment (start 116.6 64.925) (end 159.7 64.925) (width 0.25) (layer "F.Cu") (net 1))
 (segment (start 150.79 125.675) (end 150.79 122.51) (width 0.25) (layer "F.Cu") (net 1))
 (segment (start 131.74 86.49) (end 131.775 86.525) (width 0.25) (layer "F.Cu") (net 1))
 (segment (start 144.03 122.52) (end 144.05 122.5) (width 0.25) (layer "F.Cu") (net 1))
 (segment (start 163.375 114.9) (end 163.4 114.875) (width 0.25) (layer "F.Cu") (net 1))
 (segment (start 159.7 64.925) (end 159.75 64.875) (width 0.25) (layer "F.Cu") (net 1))
 (segment (start 159.75 64.875) (end 159.75 86.475) (width 0.254) (layer "F.Cu") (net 1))
 (segment (start 116.55 64.975) (end 116.6 64.925) (width 0.25) (layer "F.Cu") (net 1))
 (segment (start 141.68 110.25) (end 141.68 114.88) (width 0.508) (layer "F.Cu") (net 1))
 (segment (start 121.9 122.525) (end 129.475 122.525) (width 0.25) (layer "F.Cu") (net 1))
 (segment (start 113.825 76.845) (end 116.43 76.845) (width 0.25) (layer "F.Cu") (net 1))
 (segment (start 159.75 55.65) (end 159.75 61.35) (width 0.25) (layer "F.Cu") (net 1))
 (segment (start 150.79 122.51) (end 150.8 122.5) (width 0.25) (layer "F.Cu") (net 1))
 (segment (start 129.475 122.525) (end 144.025 122.525) (width 0.25) (layer "F.Cu") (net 1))
 (segment (start 144.03 125.675) (end 144.03 122.52) (width 0.25) (layer "F.Cu") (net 1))
 (segment (start 144.05 122.5) (end 150.8 122.5) (width 0.25) (layer "F.Cu") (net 1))
 (segment (start 116.55 76.725) (end 116.55 64.975) (width 0.25) (layer "F.Cu") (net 1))
 (via (at 159.75 55.65) (size 0.8) (drill 0.4) (layers "F.Cu" "B.Cu") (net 1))
 (segment (start 159.75 55.65) (end 159.72 55.68) (width 0.25) (layer "B.Cu") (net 1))
 (segment (start 159.72 55.68) (end 149.39 55.68) (width 0.25) (layer "B.Cu") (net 1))
 (segment (start 140.405 56.855) (end 139.23 55.68) (width 0.25) (layer "B.Cu") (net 24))
 (segment (start 140.405 62.21) (end 140.405 56.855) (width 0.25) (layer "B.Cu") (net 24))
 (segment (start 146.98 68.785) (end 140.405 62.21) (width 0.25) (layer "B.Cu") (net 24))
 (segment (start 139.23 63.555) (end 139.23 58.22) (width 0.25) (layer "B.Cu") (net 23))
 (segment (start 144.44 68.785) (end 139.25 63.595) (width 0.25) (layer "B.Cu") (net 23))
 (segment (start 139.25 63.575) (end 139.23 63.555) (width 0.25) (layer "B.Cu") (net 23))
 (segment (start 139.25 63.595) (end 139.25 63.575) (width 0.25) (layer "B.Cu") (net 23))
 (segment (start 137.865 56.855) (end 136.69 55.68) (width 0.25) (layer "B.Cu") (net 22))
 (segment (start 137.865 64.75) (end 137.865 56.855) (width 0.25) (layer "B.Cu") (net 22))
 (segment (start 141.9 68.785) (end 137.865 64.75) (width 0.25) (layer "B.Cu") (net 22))
 (segment (start 136.69 65.215) (end 136.69 58.22) (width 0.25) (layer "B.Cu") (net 21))
 (segment (start 136.725 66.15) (end 136.725 65.25) (width 0.25) (layer "B.Cu") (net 21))
 (segment (start 136.725 65.25) (end 136.69 65.215) (width 0.25) (layer "B.Cu") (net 21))
 (segment (start 139.36 68.785) (end 136.725 66.15) (width 0.25) (layer "B.Cu") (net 21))
 (segment (start 135.325 56.855) (end 134.15 55.68) (width 0.25) (layer "B.Cu") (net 20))
 (segment (start 136.82 68.785) (end 135.325 67.29) (width 0.25) (layer "B.Cu") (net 20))
 (segment (start 135.325 67.29) (end 135.325 56.855) (width 0.25) (layer "B.Cu") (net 20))
 (segment (start 134.28 58.35) (end 134.15 58.22) (width 0.25) (layer "B.Cu") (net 19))
 (segment (start 134.28 68.785) (end 134.28 58.35) (width 0.25) (layer "B.Cu") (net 19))
 (segment (start 132.785 67.74) (end 132.785 56.855) (width 0.25) (layer "B.Cu") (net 18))
 (segment (start 132.785 56.855) (end 131.61 55.68) (width 0.25) (layer "B.Cu") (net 18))
 (segment (start 131.74 68.785) (end 132.785 67.74) (width 0.25) (layer "B.Cu") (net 18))
 (segment (start 131.61 66.375) (end 131.61 58.22) (width 0.25) (layer "B.Cu") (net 17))
 (segment (start 129.2 68.785) (end 131.61 66.375) (width 0.25) (layer "B.Cu") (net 17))
 (segment (start 130.245 56.855) (end 129.07 55.68) (width 0.25) (layer "B.Cu") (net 16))
 (segment (start 126.66 68.785) (end 130.245 65.2) (width 0.25) (layer "B.Cu") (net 16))
 (segment (start 130.245 65.2) (end 130.245 56.855) (width 0.25) (layer "B.Cu") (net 16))
 (segment (start 124.12 68.785) (end 129.07 63.835) (width 0.25) (layer "B.Cu") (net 15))
 (segment (start 129.07 63.835) (end 129.07 58.22) (width 0.25) (layer "B.Cu") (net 15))
 (segment (start 121.58 68.785) (end 127.705 62.66) (width 0.25) (layer "B.Cu") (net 14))
 (segment (start 127.705 62.66) (end 127.705 56.855) (width 0.25) (layer "B.Cu") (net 14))
 (segment (start 127.705 56.855) (end 126.53 55.68) (width 0.25) (layer "B.Cu") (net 14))
 (segment (start 119.04 65.71) (end 126.53 58.22) (width 0.25) (layer "B.Cu") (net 13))
 (segment (start 119.04 68.785) (end 119.04 65.71) (width 0.25) (layer "B.Cu") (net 13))
 (segment (start 153.255 125.6) (end 153.255 98.965) (width 0.25) (layer "B.Cu") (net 10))
 (segment (start 153.33 125.675) (end 153.255 125.6) (width 0.25) (layer "B.Cu") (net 10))
 (segment (start 153.255 98.965) (end 149.3 95.01) (width 0.25) (layer "B.Cu") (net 10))
 (segment (start 139.475 112.2) (end 137.725 110.45) (width 0.25) (layer "F.Cu") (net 9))
 (segment (start 137.725 103.755) (end 128.98 95.01) (width 0.25) (layer "F.Cu") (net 9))
 (segment (start 139.475 120) (end 139.475 112.2) (width 0.25) (layer "F.Cu") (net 9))
 (segment (start 139.525 120.05) (end 139.475 120) (width 0.25) (layer "F.Cu") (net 9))
 (segment (start 137.725 110.45) (end 137.725 103.755) (width 0.25) (layer "F.Cu") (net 9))
 (segment (start 155.875 120.05) (end 139.525 120.05) (width 0.25) (layer "F.Cu") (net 9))
 (via (at 155.875 120.05) (size 0.8) (drill 0.4) (layers "F.Cu" "B.Cu") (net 9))
 (segment (start 155.87 120.095) (end 155.875 120.1) (width 0.25) (layer "B.Cu") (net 9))
 (segment (start 155.875 120.1) (end 155.875 120.05) (width 0.25) (layer "B.Cu") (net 9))
 (segment (start 155.825 120.05) (end 155.85 120.075) (width 0.25) (layer "B.Cu") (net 9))
 (segment (start 155.875 120.05) (end 155.825 120.05) (width 0.25) (layer "B.Cu") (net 9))
 (segment (start 155.87 125.675) (end 155.87 120.095) (width 0.25) (layer "B.Cu") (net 9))
 (segment (start 133.55 115) (end 132.935 114.385) (width 0.25) (layer "F.Cu") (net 7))
 (segment (start 132.935 114.385) (end 132.935 101.505) (width 0.25) (layer "F.Cu") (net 7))
 (segment (start 132.935 101.505) (end 126.44 95.01) (width 0.25) (layer "F.Cu") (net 7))
 (via (at 133.55 115) (size 0.8) (drill 0.4) (layers "F.Cu" "B.Cu") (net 7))
 (segment (start 133.55 115) (end 133.55 115.025) (width 0.25) (layer "B.Cu") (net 7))
 (segment (start 133.55 122.815) (end 133.55 115) (width 0.25) (layer "B.Cu") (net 7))
 (segment (start 136.41 125.675) (end 133.55 122.815) (width 0.25) (layer "B.Cu") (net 7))
 (segment (start 128.95 89.95) (end 128.95 89.96) (width 0.25) (layer "B.Cu") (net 34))
 (segment (start 144.44 84.025) (end 138.515 89.95) (width 0.25) (layer "B.Cu") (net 34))
 (segment (start 128.95 89.96) (end 123.9 95.01) (width 0.25) (layer "B.Cu") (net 34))
 (segment (start 138.515 89.95) (end 128.95 89.95) (width 0.25) (layer "B.Cu") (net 34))
 (segment (start 137.225 88.7) (end 127.67 88.7) (width 0.25) (layer "B.Cu") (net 33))
 (segment (start 127.67 88.7) (end 121.36 95.01) (width 0.25) (layer "B.Cu") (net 33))
 (segment (start 141.9 84.025) (end 137.225 88.7) (width 0.25) (layer "B.Cu") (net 33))
 (segment (start 126.15 87.68) (end 118.82 95.01) (width 0.25) (layer "B.Cu") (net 32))
 (segment (start 139.36 84.025) (end 135.71 87.675) (width 0.25) (layer "B.Cu") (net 32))
 (segment (start 126.15 87.675) (end 126.15 87.68) (width 0.25) (layer "B.Cu") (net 32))
 (segment (start 135.71 87.675) (end 126.15 87.675) (width 0.25) (layer "B.Cu") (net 32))
 (segment (start 124.765 86.525) (end 116.28 95.01) (width 0.25) (layer "B.Cu") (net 31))
 (segment (start 136.82 84.025) (end 134.32 86.525) (width 0.25) (layer "B.Cu") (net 31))
 (segment (start 134.32 86.525) (end 124.765 86.525) (width 0.25) (layer "B.Cu") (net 31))
 (segment (start 135.88 91.75) (end 139.14 95.01) (width 0.25) (layer "F.Cu") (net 11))
 (segment (start 113.825 79.385) (end 116.49 79.385) (width 0.25) (layer "F.Cu") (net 11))
 (segment (start 117.475 91.75) (end 135.88 91.75) (width 0.25) (layer "F.Cu") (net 11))
 (segment (start 116.575 79.3) (end 116.575 90.85) (width 0.25) (layer "F.Cu") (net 11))
 (segment (start 116.575 90.85) (end 117.475 91.75) (width 0.25) (layer "F.Cu") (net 11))
 (segment (start 116.49 79.385) (end 116.575 79.3) (width 0.25) (layer "F.Cu") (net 11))
 (segment (start 134.265 92.675) (end 136.6 95.01) (width 0.25) (layer "F.Cu") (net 12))
 (segment (start 113.825 81.925) (end 113.825 91.325) (width 0.25) (layer "F.Cu") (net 12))
 (segment (start 115.175 92.675) (end 134.265 92.675) (width 0.25) (layer "F.Cu") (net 12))
 (segment (start 113.825 91.325) (end 115.175 92.675) (width 0.25) (layer "F.Cu") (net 12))
 (segment (start 137.775 116.8) (end 132.99 116.8) (width 0.25) (layer "F.Cu") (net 5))
 (segment (start 132.99 116.8) (end 126.44 110.25) (width 0.25) (layer "F.Cu") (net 5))
 (via (at 137.775 116.8) (size 0.8) (drill 0.4) (layers "F.Cu" "B.Cu") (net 5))
 (segment (start 141.525 116.825) (end 141.5 116.8) (width 0.25) (layer "B.Cu") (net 5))
 (segment (start 141.49 125.675) (end 141.49 116.86) (width 0.25) (layer "B.Cu") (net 5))
 (segment (start 141.49 116.86) (end 141.525 116.825) (width 0.25) (layer "B.Cu") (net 5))
 (segment (start 141.5 116.8) (end 137.775 116.8) (width 0.25) (layer "B.Cu") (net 5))
 (segment (start 137.775 116.8) (end 137.825 116.8) (width 0.25) (layer "B.Cu") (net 5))
 (segment (start 134.875 108.725) (end 125.425 108.725) (width 0.25) (layer "B.Cu") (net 6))
 (segment (start 125.425 108.725) (end 123.9 110.25) (width 0.25) (layer "B.Cu") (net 6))
 (segment (start 138.95 125.675) (end 135.185 121.91) (width 0.25) (layer "B.Cu") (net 6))
 (segment (start 135.185 121.91) (end 135.185 109.035) (width 0.25) (layer "B.Cu") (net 6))
 (segment (start 135.185 109.035) (end 134.875 108.725) (width 0.25) (layer "B.Cu") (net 6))
 (segment (start 126.96 120.94) (end 131.52 116.38) (width 0.25) (layer "B.Cu") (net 2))
 (segment (start 131.52 116.38) (end 131.52 110.25) (width 0.25) (layer "B.Cu") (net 2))
 (segment (start 126.96 125.745) (end 126.96 120.94) (width 0.25) (layer "B.Cu") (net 2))
 (segment (start 119.34 121.51) (end 128.98 111.87) (width 0.25) (layer "B.Cu") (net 4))
 (segment (start 119.34 125.745) (end 119.34 121.51) (width 0.25) (layer "B.Cu") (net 4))
 (segment (start 128.98 111.87) (end 128.98 110.25) (width 0.25) (layer "B.Cu") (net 4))
 (segment (start 159.7 113.025) (end 159.7 97.525) (width 0.25) (layer "F.Cu") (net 8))
 (segment (start 136.55 97.5) (end 134.06 95.01) (width 0.25) (layer "F.Cu") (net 8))
 (segment (start 159.675 97.5) (end 136.55 97.5) (width 0.25) (layer "F.Cu") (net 8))
 (segment (start 159.7 97.525) (end 159.675 97.5) (width 0.25) (layer "F.Cu") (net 8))
 (via (at 159.7 113.025) (size 0.8) (drill 0.4) (layers "F.Cu" "B.Cu") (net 8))
 (segment (start 158.41 120.185) (end 158.41 125.675) (width 0.25) (layer "B.Cu") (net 8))
 (segment (start 159.7 113.025) (end 158.4 114.325) (width 0.25) (layer "B.Cu") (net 8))
 (segment (start 158.4 114.325) (end 158.4 120.175) (width 0.25) (layer "B.Cu") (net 8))
 (segment (start 140.305 90.7) (end 128.869009 90.7) (width 0.25) (layer "B.Cu") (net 35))
 (segment (start 125.025 94.544009) (end 125.025 98.525) (width 0.25) (layer "B.Cu") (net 35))
 (segment (start 128.869009 90.7) (end 125.025 94.544009) (width 0.25) (layer "B.Cu") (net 35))
 (segment (start 146.98 84.025) (end 140.305 90.7) (width 0.25) (layer "B.Cu") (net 35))
 (segment (start 125.025 98.525) (end 121.35 98.525) (width 0.25) (layer "B.Cu") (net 35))
 (segment (start 121.35 98.525) (end 121.36 98.535) (width 0.25) (layer "B.Cu") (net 35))
 (segment (start 121.36 98.535) (end 121.36 110.25) (width 0.25) (layer "B.Cu") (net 35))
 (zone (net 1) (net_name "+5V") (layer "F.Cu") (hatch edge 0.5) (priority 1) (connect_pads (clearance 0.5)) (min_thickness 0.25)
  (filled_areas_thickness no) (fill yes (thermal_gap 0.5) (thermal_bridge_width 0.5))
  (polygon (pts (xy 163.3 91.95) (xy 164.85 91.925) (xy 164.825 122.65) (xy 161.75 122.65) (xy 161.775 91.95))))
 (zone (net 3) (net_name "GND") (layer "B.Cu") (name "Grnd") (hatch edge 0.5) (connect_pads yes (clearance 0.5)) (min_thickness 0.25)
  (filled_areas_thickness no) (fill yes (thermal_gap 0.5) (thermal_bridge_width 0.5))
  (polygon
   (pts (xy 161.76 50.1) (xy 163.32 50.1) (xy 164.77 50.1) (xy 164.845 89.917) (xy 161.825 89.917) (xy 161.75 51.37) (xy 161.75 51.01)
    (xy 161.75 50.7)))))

